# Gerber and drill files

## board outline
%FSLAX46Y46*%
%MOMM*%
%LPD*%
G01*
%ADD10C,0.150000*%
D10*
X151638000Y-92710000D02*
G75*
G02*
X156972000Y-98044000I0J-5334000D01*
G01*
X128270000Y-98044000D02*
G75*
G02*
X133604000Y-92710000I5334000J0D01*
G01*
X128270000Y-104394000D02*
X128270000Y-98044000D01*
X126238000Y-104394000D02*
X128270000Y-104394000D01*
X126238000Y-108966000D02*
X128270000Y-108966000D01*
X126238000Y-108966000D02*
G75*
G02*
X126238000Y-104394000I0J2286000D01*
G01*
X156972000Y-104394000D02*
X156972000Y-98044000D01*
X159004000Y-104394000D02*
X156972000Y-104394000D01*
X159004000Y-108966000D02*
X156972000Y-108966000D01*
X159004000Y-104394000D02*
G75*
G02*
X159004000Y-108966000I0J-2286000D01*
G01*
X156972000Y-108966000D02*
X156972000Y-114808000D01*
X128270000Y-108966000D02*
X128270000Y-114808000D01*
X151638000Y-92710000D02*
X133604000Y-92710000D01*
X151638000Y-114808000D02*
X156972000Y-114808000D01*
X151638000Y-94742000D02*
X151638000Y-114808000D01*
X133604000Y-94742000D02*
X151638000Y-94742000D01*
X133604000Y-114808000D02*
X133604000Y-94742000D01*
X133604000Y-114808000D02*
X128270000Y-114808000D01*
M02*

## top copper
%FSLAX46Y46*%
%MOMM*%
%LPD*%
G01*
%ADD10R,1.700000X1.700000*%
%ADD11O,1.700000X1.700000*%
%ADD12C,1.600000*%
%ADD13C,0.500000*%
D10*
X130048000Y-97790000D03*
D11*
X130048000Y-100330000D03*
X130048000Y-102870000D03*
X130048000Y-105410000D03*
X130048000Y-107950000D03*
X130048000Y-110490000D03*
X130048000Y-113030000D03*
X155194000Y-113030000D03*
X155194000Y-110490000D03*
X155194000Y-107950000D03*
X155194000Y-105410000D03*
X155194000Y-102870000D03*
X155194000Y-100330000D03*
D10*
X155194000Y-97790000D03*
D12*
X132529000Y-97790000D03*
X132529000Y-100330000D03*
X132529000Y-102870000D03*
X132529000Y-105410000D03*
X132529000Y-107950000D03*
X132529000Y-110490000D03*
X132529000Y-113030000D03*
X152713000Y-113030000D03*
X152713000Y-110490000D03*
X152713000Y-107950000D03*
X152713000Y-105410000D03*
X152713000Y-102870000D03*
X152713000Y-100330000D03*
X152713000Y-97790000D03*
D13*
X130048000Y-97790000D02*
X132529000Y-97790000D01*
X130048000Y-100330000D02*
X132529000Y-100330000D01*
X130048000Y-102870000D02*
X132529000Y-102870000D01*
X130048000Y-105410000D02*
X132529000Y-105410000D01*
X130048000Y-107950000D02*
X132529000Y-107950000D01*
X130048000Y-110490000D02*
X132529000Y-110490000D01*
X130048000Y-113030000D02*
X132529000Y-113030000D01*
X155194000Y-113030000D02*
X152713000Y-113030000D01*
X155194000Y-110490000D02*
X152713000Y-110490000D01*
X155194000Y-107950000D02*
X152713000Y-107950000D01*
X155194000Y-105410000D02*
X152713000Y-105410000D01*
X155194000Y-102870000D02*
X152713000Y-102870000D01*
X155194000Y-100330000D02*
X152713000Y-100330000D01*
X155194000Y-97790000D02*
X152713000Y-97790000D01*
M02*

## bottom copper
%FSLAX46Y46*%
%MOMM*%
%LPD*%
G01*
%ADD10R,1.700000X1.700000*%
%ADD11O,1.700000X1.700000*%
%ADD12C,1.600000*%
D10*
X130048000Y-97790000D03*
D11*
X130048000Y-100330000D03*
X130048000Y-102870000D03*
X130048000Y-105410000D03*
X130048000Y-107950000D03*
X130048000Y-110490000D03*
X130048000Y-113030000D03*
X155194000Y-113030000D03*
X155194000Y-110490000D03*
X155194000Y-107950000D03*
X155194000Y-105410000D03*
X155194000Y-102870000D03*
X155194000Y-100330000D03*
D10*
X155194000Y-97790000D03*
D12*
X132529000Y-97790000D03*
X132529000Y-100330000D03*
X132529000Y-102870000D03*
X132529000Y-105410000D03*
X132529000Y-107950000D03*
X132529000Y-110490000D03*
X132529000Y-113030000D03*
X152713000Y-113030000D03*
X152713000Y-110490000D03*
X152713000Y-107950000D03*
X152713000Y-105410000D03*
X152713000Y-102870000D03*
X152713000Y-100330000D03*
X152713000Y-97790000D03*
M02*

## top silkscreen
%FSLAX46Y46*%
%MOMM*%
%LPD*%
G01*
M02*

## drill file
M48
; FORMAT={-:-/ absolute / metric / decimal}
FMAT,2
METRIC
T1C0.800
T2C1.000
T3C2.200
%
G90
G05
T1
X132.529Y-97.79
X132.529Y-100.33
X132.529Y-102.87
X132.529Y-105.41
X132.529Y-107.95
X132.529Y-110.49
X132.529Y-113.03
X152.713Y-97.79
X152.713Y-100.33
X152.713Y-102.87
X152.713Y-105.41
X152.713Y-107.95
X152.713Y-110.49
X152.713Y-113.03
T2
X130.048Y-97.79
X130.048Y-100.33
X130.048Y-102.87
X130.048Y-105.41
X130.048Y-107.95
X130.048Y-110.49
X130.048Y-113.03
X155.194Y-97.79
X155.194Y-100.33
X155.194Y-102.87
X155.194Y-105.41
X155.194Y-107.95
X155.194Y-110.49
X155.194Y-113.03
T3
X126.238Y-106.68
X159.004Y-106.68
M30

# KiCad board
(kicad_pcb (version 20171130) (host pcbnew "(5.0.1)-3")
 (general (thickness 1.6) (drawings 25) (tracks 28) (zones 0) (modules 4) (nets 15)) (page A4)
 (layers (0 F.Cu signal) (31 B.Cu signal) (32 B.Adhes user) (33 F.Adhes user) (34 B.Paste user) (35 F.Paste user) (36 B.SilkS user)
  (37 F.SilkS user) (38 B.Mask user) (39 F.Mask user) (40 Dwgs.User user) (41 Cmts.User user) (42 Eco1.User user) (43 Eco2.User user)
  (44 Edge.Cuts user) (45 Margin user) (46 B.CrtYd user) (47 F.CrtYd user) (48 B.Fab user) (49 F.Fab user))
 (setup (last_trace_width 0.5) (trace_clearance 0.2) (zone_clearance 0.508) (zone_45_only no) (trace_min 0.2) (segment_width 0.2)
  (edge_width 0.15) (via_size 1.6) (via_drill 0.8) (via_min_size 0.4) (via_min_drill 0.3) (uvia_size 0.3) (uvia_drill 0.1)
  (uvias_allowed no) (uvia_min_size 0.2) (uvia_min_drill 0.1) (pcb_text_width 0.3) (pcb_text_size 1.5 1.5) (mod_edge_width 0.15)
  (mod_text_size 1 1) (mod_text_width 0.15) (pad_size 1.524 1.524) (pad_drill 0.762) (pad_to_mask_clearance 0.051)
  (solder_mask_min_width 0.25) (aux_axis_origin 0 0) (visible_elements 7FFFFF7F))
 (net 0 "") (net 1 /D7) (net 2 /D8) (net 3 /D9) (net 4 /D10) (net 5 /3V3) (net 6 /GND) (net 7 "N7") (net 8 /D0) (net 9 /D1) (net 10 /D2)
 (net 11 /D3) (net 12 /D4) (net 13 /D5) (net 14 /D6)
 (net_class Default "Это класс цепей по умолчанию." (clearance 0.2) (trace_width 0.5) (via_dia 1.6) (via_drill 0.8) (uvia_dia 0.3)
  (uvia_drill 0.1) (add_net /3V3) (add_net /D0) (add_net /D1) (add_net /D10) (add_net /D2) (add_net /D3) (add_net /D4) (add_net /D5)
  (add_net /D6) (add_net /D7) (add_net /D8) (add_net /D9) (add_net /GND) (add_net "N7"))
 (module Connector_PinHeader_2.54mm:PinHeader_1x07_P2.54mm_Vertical (layer B.Cu) (at 130.048 97.79 180)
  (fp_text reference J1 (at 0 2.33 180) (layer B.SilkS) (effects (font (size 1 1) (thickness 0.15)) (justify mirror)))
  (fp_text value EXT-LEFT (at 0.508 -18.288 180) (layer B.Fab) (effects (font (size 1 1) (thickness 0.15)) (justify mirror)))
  (pad 1 thru_hole rect (at 0 0 180) (size 1.7 1.7) (drill 1) (layers *.Cu *.Mask) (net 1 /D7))
  (pad 2 thru_hole oval (at 0 -2.54 180) (size 1.7 1.7) (drill 1) (layers *.Cu *.Mask) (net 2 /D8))
  (pad 3 thru_hole oval (at 0 -5.08 180) (size 1.7 1.7) (drill 1) (layers *.Cu *.Mask) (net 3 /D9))
  (pad 4 thru_hole oval (at 0 -7.62 180) (size 1.7 1.7) (drill 1) (layers *.Cu *.Mask) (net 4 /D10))
  (pad 5 thru_hole oval (at 0 -10.16 180) (size 1.7 1.7) (drill 1) (layers *.Cu *.Mask) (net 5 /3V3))
  (pad 6 thru_hole oval (at 0 -12.7 180) (size 1.7 1.7) (drill 1) (layers *.Cu *.Mask) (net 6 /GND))
  (pad 7 thru_hole oval (at 0 -15.24 180) (size 1.7 1.7) (drill 1) (layers *.Cu *.Mask) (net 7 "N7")))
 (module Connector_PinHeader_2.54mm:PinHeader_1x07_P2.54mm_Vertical (layer B.Cu) (at 155.194 97.79 180)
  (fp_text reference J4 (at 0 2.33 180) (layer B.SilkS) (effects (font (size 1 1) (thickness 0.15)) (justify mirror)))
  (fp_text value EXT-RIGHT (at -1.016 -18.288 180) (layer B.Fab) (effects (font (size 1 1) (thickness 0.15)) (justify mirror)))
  (pad 7 thru_hole oval (at 0 -15.24 180) (size 1.7 1.7) (drill 1) (layers *.Cu *.Mask) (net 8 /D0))
  (pad 6 thru_hole oval (at 0 -12.7 180) (size 1.7 1.7) (drill 1) (layers *.Cu *.Mask) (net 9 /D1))
  (pad 5 thru_hole oval (at 0 -10.16 180) (size 1.7 1.7) (drill 1) (layers *.Cu *.Mask) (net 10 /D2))
  (pad 4 thru_hole oval (at 0 -7.62 180) (size 1.7 1.7) (drill 1) (layers *.Cu *.Mask) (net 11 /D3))
  (pad 3 thru_hole oval (at 0 -5.08 180) (size 1.7 1.7) (drill 1) (layers *.Cu *.Mask) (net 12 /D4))
  (pad 2 thru_hole oval (at 0 -2.54 180) (size 1.7 1.7) (drill 1) (layers *.Cu *.Mask) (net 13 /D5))
  (pad 1 thru_hole rect (at 0 0 180) (size 1.7 1.7) (drill 1) (layers *.Cu *.Mask) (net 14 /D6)))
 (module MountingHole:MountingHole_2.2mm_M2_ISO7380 (layer F.Cu) (at 126.238 106.68)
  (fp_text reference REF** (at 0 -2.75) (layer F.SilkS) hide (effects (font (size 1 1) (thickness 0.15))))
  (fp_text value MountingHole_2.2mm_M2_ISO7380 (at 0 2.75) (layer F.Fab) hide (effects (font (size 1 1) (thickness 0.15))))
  (pad 1 np_thru_hole circle (at 0 0) (size 2.2 2.2) (drill 2.2) (layers *.Cu *.Mask)))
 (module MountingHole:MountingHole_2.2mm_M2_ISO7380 (layer F.Cu) (at 159.004 106.68)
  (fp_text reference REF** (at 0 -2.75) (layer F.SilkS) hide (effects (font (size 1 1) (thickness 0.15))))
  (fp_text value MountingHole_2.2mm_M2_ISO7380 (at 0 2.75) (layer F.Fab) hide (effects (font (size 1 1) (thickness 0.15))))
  (pad 1 np_thru_hole circle (at 0 0) (size 2.2 2.2) (drill 2.2) (layers *.Cu *.Mask)))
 (gr_arc (start 151.638 98.044) (end 156.972 98.044) (angle -90) (layer Edge.Cuts) (width 0.15))
 (gr_arc (start 133.604 98.044) (end 133.604 92.71) (angle -90) (layer Edge.Cuts) (width 0.15))
 (gr_line (start 128.27 104.394) (end 128.27 98.044) (layer Edge.Cuts) (width 0.15))
 (gr_line (start 126.238 104.394) (end 128.27 104.394) (layer Edge.Cuts) (width 0.15))
 (gr_line (start 126.238 108.966) (end 128.27 108.966) (layer Edge.Cuts) (width 0.15))
 (gr_arc (start 126.238 106.68) (end 126.238 104.394) (angle -180) (layer Edge.Cuts) (width 0.15))
 (gr_line (start 156.972 104.394) (end 156.972 98.044) (layer Edge.Cuts) (width 0.15))
 (gr_line (start 159.004 104.394) (end 156.972 104.394) (layer Edge.Cuts) (width 0.15))
 (gr_line (start 159.004 108.966) (end 156.972 108.966) (layer Edge.Cuts) (width 0.15))
 (gr_arc (start 159.004 106.68) (end 159.004 108.966) (angle -180) (layer Edge.Cuts) (width 0.15))
 (gr_line (start 156.972 108.966) (end 156.972 114.808) (layer Edge.Cuts) (width 0.15))
 (gr_line (start 128.27 108.966) (end 128.27 114.808) (layer Edge.Cuts) (width 0.15))
 (gr_line (start 151.638 92.71) (end 133.604 92.71) (layer Edge.Cuts) (width 0.15))
 (gr_line (start 151.638 114.808) (end 156.972 114.808) (layer Edge.Cuts) (width 0.15))
 (gr_line (start 151.638 94.742) (end 151.638 114.808) (layer Edge.Cuts) (width 0.15))
 (gr_line (start 133.604 94.742) (end 151.638 94.742) (layer Edge.Cuts) (width 0.15))
 (gr_line (start 133.604 114.808) (end 133.604 94.742) (layer Edge.Cuts) (width 0.15))
 (gr_line (start 133.604 114.808) (end 128.27 114.808) (layer Edge.Cuts) (width 0.15))
 (via (at 132.529 97.79) (size 1.6) (drill 0.8) (layers F.Cu B.Cu) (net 1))
 (segment (start 130.048 97.79) (end 132.529 97.79) (width 0.5) (layer F.Cu) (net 1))
 (via (at 132.529 100.33) (size 1.6) (drill 0.8) (layers F.Cu B.Cu) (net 2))
 (segment (start 130.048 100.33) (end 132.529 100.33) (width 0.5) (layer F.Cu) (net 2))
 (via (at 132.529 102.87) (size 1.6) (drill 0.8) (layers F.Cu B.Cu) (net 3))
 (segment (start 130.048 102.87) (end 132.529 102.87) (width 0.5) (layer F.Cu) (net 3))
 (via (at 132.529 105.41) (size 1.6) (drill 0.8) (layers F.Cu B.Cu) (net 4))
 (segment (start 130.048 105.41) (end 132.529 105.41) (width 0.5) (layer F.Cu) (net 4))
 (via (at 132.529 107.95) (size 1.6) (drill 0.8) (layers F.Cu B.Cu) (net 5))
 (segment (start 130.048 107.95) (end 132.529 107.95) (width 0.5) (layer F.Cu) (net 5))
 (via (at 132.529 110.49) (size 1.6) (drill 0.8) (layers F.Cu B.Cu) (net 6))
 (segment (start 130.048 110.49) (end 132.529 110.49) (width 0.5) (layer F.Cu) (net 6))
 (via (at 132.529 113.03) (size 1.6) (drill 0.8) (layers F.Cu B.Cu) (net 7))
 (segment (start 130.048 113.03) (end 132.529 113.03) (width 0.5) (layer F.Cu) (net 7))
 (via (at 152.713 113.03) (size 1.6) (drill 0.8) (layers F.Cu B.Cu) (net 8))
 (segment (start 155.194 113.03) (end 152.713 113.03) (width 0.5) (layer F.Cu) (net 8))
 (via (at 152.713 110.49) (size 1.6) (drill 0.8) (layers F.Cu B.Cu) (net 9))
 (segment (start 155.194 110.49) (end 152.713 110.49) (width 0.5) (layer F.Cu) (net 9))
 (via (at 152.713 107.95) (size 1.6) (drill 0.8) (layers F.Cu B.Cu) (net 10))
 (segment (start 155.194 107.95) (end 152.713 107.95) (width 0.5) (layer F.Cu) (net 10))
 (via (at 152.713 105.41) (size 1.6) (drill 0.8) (layers F.Cu B.Cu) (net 11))
 (segment (start 155.194 105.41) (end 152.713 105.41) (width 0.5) (layer F.Cu) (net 11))
 (via (at 152.713 102.87) (size 1.6) (drill 0.8) (layers F.Cu B.Cu) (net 12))
 (segment (start 155.194 102.87) (end 152.713 102.87) (width 0.5) (layer F.Cu) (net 12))
 (via (at 152.713 100.33) (size 1.6) (drill 0.8) (layers F.Cu B.Cu) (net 13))
 (segment (start 155.194 100.33) (end 152.713 100.33) (width 0.5) (layer F.Cu) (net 13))
 (via (at 152.713 97.79) (size 1.6) (drill 0.8) (layers F.Cu B.Cu) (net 14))
 (segment (start 155.194 97.79) (end 152.713 97.79) (width 0.5) (layer F.Cu) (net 14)))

